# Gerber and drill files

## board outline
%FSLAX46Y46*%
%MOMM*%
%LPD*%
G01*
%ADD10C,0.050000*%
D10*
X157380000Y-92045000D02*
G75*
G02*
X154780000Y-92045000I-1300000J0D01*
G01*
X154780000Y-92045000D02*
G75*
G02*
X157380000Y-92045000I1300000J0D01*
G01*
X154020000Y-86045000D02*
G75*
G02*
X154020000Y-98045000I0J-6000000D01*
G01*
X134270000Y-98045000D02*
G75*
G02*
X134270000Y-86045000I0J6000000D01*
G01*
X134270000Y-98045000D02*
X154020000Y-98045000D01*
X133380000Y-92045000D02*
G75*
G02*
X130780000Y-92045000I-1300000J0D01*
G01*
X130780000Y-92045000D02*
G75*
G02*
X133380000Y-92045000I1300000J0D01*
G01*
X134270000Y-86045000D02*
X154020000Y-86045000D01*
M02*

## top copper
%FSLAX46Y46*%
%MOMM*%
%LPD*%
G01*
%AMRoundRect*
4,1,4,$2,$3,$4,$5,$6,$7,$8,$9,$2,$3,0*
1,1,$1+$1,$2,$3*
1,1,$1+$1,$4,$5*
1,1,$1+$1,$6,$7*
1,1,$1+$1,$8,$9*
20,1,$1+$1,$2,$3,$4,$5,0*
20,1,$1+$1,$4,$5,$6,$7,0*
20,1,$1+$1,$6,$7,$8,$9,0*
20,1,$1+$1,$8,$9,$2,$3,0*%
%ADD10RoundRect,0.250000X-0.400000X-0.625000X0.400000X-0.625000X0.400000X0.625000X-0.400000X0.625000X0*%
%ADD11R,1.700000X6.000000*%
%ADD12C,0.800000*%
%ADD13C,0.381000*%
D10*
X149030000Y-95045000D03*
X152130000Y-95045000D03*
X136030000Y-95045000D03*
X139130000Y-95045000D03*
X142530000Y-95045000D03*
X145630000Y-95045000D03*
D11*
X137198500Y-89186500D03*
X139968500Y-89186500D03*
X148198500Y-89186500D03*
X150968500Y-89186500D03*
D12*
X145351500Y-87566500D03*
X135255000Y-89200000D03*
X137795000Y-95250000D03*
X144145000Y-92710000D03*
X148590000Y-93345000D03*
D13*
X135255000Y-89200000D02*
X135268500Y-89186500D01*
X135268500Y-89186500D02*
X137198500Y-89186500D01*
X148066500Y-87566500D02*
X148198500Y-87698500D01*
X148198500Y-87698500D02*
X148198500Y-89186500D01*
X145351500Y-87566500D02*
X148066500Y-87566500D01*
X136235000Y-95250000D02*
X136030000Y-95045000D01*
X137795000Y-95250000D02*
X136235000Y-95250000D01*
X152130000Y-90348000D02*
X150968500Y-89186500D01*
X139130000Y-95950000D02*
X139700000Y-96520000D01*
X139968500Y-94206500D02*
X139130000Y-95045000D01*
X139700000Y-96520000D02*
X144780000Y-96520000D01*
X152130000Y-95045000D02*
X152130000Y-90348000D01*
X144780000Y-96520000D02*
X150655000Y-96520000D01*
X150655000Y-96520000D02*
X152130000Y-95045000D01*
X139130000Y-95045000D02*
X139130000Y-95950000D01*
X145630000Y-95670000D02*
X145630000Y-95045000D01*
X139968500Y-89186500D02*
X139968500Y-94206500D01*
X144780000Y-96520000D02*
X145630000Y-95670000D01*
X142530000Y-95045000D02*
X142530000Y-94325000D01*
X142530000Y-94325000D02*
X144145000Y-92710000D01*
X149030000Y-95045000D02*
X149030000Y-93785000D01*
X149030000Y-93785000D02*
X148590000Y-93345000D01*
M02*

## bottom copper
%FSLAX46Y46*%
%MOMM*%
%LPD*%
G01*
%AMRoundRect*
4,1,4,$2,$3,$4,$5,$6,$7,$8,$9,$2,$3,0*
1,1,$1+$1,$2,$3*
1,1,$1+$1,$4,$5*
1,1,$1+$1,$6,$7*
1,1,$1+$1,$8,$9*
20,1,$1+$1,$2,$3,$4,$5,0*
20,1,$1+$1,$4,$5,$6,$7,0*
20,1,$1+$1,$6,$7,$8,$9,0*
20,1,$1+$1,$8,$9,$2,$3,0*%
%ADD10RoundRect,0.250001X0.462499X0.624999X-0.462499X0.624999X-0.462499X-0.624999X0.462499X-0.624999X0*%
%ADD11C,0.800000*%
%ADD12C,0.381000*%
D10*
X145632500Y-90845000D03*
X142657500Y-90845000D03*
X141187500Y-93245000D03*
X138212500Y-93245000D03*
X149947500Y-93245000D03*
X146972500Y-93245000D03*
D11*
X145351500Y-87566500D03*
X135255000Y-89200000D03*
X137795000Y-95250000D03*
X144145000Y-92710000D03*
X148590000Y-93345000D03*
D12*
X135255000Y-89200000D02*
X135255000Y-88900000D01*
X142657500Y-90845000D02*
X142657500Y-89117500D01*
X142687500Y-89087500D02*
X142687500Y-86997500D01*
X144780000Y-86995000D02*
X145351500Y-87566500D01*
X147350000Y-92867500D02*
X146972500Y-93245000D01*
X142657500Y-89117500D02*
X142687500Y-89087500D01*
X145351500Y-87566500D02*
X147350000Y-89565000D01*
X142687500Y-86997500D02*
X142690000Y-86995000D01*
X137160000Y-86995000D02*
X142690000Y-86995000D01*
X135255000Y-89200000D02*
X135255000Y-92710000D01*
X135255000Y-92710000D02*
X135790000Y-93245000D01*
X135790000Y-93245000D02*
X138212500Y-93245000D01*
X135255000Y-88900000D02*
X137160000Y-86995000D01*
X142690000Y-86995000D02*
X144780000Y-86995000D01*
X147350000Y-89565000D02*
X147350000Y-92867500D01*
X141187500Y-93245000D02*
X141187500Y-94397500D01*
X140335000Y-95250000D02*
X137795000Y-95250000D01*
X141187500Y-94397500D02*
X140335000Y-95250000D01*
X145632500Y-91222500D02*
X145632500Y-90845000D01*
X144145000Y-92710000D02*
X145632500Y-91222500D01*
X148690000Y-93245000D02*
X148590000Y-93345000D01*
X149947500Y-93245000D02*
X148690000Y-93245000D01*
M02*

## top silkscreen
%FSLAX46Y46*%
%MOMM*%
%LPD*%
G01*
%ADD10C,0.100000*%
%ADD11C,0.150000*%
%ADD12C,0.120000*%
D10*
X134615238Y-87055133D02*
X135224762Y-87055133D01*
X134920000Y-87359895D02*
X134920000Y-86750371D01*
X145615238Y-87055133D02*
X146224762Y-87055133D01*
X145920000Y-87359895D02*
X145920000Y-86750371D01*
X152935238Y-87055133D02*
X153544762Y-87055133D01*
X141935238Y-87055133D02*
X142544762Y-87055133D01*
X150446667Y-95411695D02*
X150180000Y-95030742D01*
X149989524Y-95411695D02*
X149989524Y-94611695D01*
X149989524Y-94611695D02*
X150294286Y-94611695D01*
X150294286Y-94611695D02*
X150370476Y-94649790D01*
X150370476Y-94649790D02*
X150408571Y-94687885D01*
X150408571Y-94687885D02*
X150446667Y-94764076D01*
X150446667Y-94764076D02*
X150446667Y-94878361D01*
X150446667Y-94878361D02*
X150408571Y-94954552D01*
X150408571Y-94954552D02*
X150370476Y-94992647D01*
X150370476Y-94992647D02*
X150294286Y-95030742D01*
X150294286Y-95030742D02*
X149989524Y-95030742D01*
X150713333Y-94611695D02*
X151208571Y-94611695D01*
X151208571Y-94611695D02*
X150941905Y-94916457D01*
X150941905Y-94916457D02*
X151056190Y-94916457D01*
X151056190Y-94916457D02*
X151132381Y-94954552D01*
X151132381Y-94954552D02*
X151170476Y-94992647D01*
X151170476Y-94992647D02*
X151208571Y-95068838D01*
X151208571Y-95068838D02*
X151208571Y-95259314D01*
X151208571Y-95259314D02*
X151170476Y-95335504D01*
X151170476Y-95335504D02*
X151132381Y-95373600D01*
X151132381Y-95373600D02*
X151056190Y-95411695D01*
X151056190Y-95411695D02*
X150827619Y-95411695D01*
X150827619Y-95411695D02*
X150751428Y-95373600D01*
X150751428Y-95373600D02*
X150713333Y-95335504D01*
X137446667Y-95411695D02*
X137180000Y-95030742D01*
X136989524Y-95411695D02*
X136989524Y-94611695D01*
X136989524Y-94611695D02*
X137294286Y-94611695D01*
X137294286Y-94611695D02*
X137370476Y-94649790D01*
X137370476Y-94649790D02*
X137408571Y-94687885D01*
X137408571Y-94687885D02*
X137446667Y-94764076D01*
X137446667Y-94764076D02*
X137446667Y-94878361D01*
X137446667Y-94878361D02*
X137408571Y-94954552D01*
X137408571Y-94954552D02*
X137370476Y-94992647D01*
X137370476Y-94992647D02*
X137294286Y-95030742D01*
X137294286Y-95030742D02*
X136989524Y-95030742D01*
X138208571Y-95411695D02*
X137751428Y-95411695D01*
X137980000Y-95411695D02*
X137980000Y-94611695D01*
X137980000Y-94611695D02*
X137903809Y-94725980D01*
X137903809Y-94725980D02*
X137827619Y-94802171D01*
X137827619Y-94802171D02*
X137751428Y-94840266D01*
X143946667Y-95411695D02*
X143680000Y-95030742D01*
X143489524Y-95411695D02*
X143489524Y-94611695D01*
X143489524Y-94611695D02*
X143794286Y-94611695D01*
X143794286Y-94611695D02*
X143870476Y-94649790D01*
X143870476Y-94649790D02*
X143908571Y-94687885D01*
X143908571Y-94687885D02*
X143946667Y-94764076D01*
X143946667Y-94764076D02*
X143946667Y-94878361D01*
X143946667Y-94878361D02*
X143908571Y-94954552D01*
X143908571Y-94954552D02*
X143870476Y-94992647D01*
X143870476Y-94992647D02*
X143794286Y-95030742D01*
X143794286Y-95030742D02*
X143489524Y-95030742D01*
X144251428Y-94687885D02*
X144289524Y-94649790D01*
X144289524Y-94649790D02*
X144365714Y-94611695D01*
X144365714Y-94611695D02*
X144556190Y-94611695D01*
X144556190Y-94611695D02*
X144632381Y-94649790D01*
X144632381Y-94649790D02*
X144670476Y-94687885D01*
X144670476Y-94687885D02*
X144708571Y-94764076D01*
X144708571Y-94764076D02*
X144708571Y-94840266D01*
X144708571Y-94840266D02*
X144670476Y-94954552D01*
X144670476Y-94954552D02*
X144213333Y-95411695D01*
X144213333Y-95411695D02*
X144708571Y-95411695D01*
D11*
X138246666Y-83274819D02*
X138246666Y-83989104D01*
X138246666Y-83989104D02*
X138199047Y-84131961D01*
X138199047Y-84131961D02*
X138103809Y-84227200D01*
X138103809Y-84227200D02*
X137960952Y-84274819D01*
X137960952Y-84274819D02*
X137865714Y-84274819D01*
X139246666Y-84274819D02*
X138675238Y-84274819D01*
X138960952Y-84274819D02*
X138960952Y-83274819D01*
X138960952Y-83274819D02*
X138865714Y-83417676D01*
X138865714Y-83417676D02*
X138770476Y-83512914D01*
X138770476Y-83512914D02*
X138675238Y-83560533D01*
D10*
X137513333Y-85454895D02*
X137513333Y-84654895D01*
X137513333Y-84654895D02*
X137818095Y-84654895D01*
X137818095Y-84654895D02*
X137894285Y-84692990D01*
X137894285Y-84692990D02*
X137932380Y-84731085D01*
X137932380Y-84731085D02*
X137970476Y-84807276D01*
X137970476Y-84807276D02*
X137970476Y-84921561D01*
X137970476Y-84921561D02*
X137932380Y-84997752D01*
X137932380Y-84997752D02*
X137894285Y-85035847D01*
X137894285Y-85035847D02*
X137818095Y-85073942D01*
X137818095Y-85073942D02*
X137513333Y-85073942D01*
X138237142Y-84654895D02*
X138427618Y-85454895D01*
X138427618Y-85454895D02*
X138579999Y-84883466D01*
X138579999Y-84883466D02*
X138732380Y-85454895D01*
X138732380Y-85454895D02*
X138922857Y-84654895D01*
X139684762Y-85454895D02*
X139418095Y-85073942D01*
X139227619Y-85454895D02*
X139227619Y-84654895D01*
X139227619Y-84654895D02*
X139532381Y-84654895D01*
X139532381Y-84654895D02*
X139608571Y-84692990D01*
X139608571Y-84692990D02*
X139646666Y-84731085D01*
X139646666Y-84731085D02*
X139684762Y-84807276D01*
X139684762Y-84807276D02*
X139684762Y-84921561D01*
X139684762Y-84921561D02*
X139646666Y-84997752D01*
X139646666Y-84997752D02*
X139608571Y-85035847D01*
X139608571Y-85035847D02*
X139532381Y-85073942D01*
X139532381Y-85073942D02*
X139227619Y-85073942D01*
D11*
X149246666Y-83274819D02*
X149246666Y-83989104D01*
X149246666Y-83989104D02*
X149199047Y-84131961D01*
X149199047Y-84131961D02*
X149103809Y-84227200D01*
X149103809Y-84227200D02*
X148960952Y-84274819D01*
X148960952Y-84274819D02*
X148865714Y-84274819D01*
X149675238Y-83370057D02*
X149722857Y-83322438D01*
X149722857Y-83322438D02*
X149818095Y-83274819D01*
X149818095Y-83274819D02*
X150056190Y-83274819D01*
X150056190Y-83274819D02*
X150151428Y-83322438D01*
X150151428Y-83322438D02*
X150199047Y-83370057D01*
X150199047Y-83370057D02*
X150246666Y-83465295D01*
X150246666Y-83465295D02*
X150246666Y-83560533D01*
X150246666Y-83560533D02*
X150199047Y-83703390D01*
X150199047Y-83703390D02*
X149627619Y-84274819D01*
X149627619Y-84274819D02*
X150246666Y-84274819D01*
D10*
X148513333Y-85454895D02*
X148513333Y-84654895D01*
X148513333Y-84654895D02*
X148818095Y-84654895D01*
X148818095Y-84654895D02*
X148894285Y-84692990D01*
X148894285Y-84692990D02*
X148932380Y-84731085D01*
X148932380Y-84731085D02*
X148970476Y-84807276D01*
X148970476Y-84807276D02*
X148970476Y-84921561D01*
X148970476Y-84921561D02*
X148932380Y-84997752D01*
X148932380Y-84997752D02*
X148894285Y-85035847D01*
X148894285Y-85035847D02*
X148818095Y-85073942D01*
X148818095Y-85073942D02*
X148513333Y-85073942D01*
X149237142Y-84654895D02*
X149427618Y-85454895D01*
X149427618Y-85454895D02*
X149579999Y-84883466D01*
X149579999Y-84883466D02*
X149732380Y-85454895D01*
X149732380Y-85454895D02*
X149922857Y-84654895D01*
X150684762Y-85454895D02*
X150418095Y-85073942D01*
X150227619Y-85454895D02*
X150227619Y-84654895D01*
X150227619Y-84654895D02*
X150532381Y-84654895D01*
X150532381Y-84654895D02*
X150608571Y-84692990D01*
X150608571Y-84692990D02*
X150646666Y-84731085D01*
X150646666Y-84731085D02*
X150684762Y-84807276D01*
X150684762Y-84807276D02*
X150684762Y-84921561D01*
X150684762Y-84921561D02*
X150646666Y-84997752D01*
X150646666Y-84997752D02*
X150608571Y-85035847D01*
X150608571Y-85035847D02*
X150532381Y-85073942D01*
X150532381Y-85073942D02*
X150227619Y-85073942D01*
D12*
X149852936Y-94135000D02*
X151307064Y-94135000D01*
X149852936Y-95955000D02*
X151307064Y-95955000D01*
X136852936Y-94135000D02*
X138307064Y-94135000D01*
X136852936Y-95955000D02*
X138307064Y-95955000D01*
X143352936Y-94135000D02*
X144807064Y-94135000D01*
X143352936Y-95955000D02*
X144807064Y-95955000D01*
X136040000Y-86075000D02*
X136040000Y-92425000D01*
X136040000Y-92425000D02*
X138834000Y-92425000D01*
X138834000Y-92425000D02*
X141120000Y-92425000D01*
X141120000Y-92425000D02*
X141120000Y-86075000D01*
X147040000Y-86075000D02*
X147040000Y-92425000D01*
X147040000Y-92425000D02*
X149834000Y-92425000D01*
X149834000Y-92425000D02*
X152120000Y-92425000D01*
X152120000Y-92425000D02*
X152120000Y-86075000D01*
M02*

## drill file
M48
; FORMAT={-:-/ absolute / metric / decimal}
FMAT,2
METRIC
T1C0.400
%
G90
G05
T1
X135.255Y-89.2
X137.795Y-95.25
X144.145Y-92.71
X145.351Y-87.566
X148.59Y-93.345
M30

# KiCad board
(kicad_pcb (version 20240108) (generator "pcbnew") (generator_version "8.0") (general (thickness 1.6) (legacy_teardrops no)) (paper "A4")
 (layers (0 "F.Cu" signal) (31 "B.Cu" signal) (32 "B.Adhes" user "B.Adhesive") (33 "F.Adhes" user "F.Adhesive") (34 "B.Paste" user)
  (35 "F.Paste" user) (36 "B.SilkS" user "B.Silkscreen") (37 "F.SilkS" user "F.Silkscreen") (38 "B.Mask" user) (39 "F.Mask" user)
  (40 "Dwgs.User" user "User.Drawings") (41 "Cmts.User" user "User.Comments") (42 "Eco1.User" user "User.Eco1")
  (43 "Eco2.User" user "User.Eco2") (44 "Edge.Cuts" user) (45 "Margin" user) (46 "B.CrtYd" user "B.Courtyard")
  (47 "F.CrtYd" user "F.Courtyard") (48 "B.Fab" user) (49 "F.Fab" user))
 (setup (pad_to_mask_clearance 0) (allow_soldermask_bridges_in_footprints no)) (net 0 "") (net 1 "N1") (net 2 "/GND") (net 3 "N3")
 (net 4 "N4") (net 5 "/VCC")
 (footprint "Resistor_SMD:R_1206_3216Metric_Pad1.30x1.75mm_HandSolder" (layer "F.Cu") (at 150.58 95.045)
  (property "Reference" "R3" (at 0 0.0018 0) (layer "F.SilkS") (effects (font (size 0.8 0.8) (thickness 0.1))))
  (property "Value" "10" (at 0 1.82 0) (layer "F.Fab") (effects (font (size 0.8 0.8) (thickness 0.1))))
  (fp_line (start -0.727064 -0.91) (end 0.727064 -0.91) (stroke (width 0.12) (type solid)) (layer "F.SilkS"))
  (fp_line (start -0.727064 0.91) (end 0.727064 0.91) (stroke (width 0.12) (type solid)) (layer "F.SilkS"))
  (pad "1" smd roundrect (at -1.55 0) (size 1.3 1.75) (layers "F.Cu" "F.Paste" "F.Mask") (roundrect_rratio 0.192308) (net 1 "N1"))
  (pad "2" smd roundrect (at 1.55 0) (size 1.3 1.75) (layers "F.Cu" "F.Paste" "F.Mask") (roundrect_rratio 0.192308) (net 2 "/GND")))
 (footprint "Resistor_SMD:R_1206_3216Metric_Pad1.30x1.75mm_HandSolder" (layer "F.Cu") (at 137.58 95.045)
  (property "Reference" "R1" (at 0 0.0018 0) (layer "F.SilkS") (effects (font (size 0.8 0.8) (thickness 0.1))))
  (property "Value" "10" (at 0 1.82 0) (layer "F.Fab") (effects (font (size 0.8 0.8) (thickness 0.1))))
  (fp_line (start -0.727064 -0.91) (end 0.727064 -0.91) (stroke (width 0.12) (type solid)) (layer "F.SilkS"))
  (fp_line (start -0.727064 0.91) (end 0.727064 0.91) (stroke (width 0.12) (type solid)) (layer "F.SilkS"))
  (pad "1" smd roundrect (at -1.55 0) (size 1.3 1.75) (layers "F.Cu" "F.Paste" "F.Mask") (roundrect_rratio 0.192308) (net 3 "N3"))
  (pad "2" smd roundrect (at 1.55 0) (size 1.3 1.75) (layers "F.Cu" "F.Paste" "F.Mask") (roundrect_rratio 0.192308) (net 2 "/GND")))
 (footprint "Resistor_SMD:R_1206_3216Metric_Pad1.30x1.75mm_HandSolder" (layer "F.Cu") (at 144.08 95.045)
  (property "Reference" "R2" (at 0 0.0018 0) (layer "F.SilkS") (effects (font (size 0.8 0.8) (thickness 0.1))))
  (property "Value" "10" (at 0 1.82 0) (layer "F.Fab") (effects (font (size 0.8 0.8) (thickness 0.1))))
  (fp_line (start -0.727064 -0.91) (end 0.727064 -0.91) (stroke (width 0.12) (type solid)) (layer "F.SilkS"))
  (fp_line (start -0.727064 0.91) (end 0.727064 0.91) (stroke (width 0.12) (type solid)) (layer "F.SilkS"))
  (pad "1" smd roundrect (at -1.55 0) (size 1.3 1.75) (layers "F.Cu" "F.Paste" "F.Mask") (roundrect_rratio 0.192308) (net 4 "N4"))
  (pad "2" smd roundrect (at 1.55 0) (size 1.3 1.75) (layers "F.Cu" "F.Paste" "F.Mask") (roundrect_rratio 0.192308) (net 2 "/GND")))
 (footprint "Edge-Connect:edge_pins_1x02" (layer "F.Cu") (at 138.58 89.25 180)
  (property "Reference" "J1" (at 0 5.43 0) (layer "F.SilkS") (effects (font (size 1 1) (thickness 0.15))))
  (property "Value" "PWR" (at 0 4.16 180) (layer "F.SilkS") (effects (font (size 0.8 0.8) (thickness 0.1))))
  (fp_line (start 2.54 3.175) (end 2.54 -3.175) (stroke (width 0.12) (type solid)) (layer "F.SilkS"))
  (fp_line (start 2.54 -3.175) (end -0.254 -3.175) (stroke (width 0.12) (type solid)) (layer "F.SilkS"))
  (fp_line (start -0.254 -3.175) (end -2.54 -3.175) (stroke (width 0.12) (type solid)) (layer "F.SilkS"))
  (fp_line (start -2.54 -3.175) (end -2.54 3.175) (stroke (width 0.12) (type solid)) (layer "F.SilkS"))
  (pad "1" smd rect (at 1.3815 0.0635) (size 1.7 6) (layers "F.Cu" "F.Paste" "F.Mask") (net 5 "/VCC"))
  (pad "2" smd rect (at -1.3885 0.0635) (size 1.7 6) (layers "F.Cu" "F.Paste" "F.Mask") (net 2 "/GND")))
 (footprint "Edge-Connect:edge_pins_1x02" (layer "F.Cu") (at 149.58 89.25 180)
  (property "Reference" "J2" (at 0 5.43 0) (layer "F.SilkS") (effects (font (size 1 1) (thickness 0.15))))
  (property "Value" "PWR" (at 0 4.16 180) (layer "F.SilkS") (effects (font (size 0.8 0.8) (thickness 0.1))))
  (fp_line (start 2.54 3.175) (end 2.54 -3.175) (stroke (width 0.12) (type solid)) (layer "F.SilkS"))
  (fp_line (start 2.54 -3.175) (end -0.254 -3.175) (stroke (width 0.12) (type solid)) (layer "F.SilkS"))
  (fp_line (start -0.254 -3.175) (end -2.54 -3.175) (stroke (width 0.12) (type solid)) (layer "F.SilkS"))
  (fp_line (start -2.54 -3.175) (end -2.54 3.175) (stroke (width 0.12) (type solid)) (layer "F.SilkS"))
  (pad "1" smd rect (at 1.3815 0.0635) (size 1.7 6) (layers "F.Cu" "F.Paste" "F.Mask") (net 5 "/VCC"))
  (pad "2" smd rect (at -1.3885 0.0635) (size 1.7 6) (layers "F.Cu" "F.Paste" "F.Mask") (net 2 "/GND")))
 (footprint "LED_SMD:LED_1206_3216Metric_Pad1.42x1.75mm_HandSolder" (layer "B.Cu") (at 144.145 90.845 180)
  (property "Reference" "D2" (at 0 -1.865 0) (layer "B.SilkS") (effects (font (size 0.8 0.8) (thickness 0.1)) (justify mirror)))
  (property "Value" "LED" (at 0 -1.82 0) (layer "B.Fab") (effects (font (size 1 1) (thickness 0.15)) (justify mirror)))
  (pad "1" smd roundrect (at -1.4875 0 180) (size 1.425 1.75) (layers "B.Cu" "B.Paste" "B.Mask") (roundrect_rratio 0.175439) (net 4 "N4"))
  (pad "2" smd roundrect (at 1.4875 0 180) (size 1.425 1.75) (layers "B.Cu" "B.Paste" "B.Mask") (roundrect_rratio 0.175439) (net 5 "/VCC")))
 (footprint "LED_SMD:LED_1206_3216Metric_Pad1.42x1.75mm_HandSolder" (layer "B.Cu") (at 139.7 93.245 180)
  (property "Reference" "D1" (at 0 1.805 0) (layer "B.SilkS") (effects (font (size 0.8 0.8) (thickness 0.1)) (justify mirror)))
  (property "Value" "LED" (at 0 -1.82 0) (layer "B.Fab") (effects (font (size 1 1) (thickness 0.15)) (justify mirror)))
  (pad "1" smd roundrect (at -1.4875 0 180) (size 1.425 1.75) (layers "B.Cu" "B.Paste" "B.Mask") (roundrect_rratio 0.175439) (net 3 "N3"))
  (pad "2" smd roundrect (at 1.4875 0 180) (size 1.425 1.75) (layers "B.Cu" "B.Paste" "B.Mask") (roundrect_rratio 0.175439) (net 5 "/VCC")))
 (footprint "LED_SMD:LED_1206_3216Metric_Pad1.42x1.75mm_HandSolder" (layer "B.Cu") (at 148.46 93.245 180)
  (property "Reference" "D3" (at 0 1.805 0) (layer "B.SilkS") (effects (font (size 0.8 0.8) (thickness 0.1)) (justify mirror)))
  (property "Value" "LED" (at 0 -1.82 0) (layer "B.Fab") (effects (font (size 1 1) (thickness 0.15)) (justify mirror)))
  (pad "1" smd roundrect (at -1.4875 0 180) (size 1.425 1.75) (layers "B.Cu" "B.Paste" "B.Mask") (roundrect_rratio 0.175439) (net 1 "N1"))
  (pad "2" smd roundrect (at 1.4875 0 180) (size 1.425 1.75) (layers "B.Cu" "B.Paste" "B.Mask") (roundrect_rratio 0.175439) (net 5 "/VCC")))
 (gr_circle (center 156.08 92.045) (end 157.38 92.045) (stroke (width 0.05) (type default)) (fill none) (layer "Edge.Cuts"))
 (gr_arc (start 154.02 86.045) (mid 160.02 92.045) (end 154.02 98.045) (stroke (width 0.05) (type default)) (layer "Edge.Cuts"))
 (gr_arc (start 134.27 98.045) (mid 128.27 92.045) (end 134.27 86.045) (stroke (width 0.05) (type default)) (layer "Edge.Cuts"))
 (gr_line (start 134.27 98.045) (end 154.02 98.045) (stroke (width 0.05) (type default)) (layer "Edge.Cuts"))
 (gr_circle (center 132.08 92.045) (end 133.38 92.045) (stroke (width 0.05) (type default)) (fill none) (layer "Edge.Cuts"))
 (gr_line (start 134.27 86.045) (end 154.02 86.045) (stroke (width 0.05) (type default)) (layer "Edge.Cuts"))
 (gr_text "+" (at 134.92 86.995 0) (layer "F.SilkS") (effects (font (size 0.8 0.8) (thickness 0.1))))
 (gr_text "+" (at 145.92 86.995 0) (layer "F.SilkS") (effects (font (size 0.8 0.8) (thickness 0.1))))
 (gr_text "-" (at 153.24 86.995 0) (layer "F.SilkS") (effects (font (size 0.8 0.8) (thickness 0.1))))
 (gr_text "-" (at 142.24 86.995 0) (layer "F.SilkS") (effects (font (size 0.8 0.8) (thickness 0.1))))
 (segment (start 135.255 89.2) (end 135.2685 89.1865) (width 0.381) (layer "F.Cu") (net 5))
 (segment (start 135.2685 89.1865) (end 137.1985 89.1865) (width 0.381) (layer "F.Cu") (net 5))
 (segment (start 148.0665 87.5665) (end 148.1985 87.6985) (width 0.381) (layer "F.Cu") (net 5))
 (segment (start 148.1985 87.6985) (end 148.1985 89.1865) (width 0.381) (layer "F.Cu") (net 5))
 (segment (start 145.3515 87.5665) (end 148.0665 87.5665) (width 0.381) (layer "F.Cu") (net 5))
 (via (at 145.3515 87.5665) (size 0.8) (drill 0.4) (layers "F.Cu" "B.Cu") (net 5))
 (via (at 135.255 89.2) (size 0.8) (drill 0.4) (layers "F.Cu" "B.Cu") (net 5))
 (segment (start 135.255 89.2) (end 135.255 88.9) (width 0.381) (layer "B.Cu") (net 5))
 (segment (start 142.6575 90.845) (end 142.6575 89.1175) (width 0.381) (layer "B.Cu") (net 5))
 (segment (start 142.6875 89.0875) (end 142.6875 86.9975) (width 0.381) (layer "B.Cu") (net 5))
 (segment (start 144.78 86.995) (end 145.3515 87.5665) (width 0.381) (layer "B.Cu") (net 5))
 (segment (start 147.35 92.8675) (end 146.9725 93.245) (width 0.381) (layer "B.Cu") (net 5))
 (segment (start 142.6575 89.1175) (end 142.6875 89.0875) (width 0.381) (layer "B.Cu") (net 5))
 (segment (start 145.3515 87.5665) (end 147.35 89.565) (width 0.381) (layer "B.Cu") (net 5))
 (segment (start 142.6875 86.9975) (end 142.69 86.995) (width 0.381) (layer "B.Cu") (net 5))
 (segment (start 137.16 86.995) (end 142.69 86.995) (width 0.381) (layer "B.Cu") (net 5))
 (segment (start 135.255 89.2) (end 135.255 92.71) (width 0.381) (layer "B.Cu") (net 5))
 (segment (start 135.255 92.71) (end 135.79 93.245) (width 0.381) (layer "B.Cu") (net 5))
 (segment (start 135.79 93.245) (end 138.2125 93.245) (width 0.381) (layer "B.Cu") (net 5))
 (segment (start 135.255 88.9) (end 137.16 86.995) (width 0.381) (layer "B.Cu") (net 5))
 (segment (start 142.69 86.995) (end 144.78 86.995) (width 0.381) (layer "B.Cu") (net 5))
 (segment (start 147.35 89.565) (end 147.35 92.8675) (width 0.381) (layer "B.Cu") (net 5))
 (segment (start 136.235 95.25) (end 136.03 95.045) (width 0.381) (layer "F.Cu") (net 3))
 (segment (start 137.795 95.25) (end 136.235 95.25) (width 0.381) (layer "F.Cu") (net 3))
 (via (at 137.795 95.25) (size 0.8) (drill 0.4) (layers "F.Cu" "B.Cu") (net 3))
 (segment (start 141.1875 93.245) (end 141.1875 94.3975) (width 0.381) (layer "B.Cu") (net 3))
 (segment (start 140.335 95.25) (end 137.795 95.25) (width 0.381) (layer "B.Cu") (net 3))
 (segment (start 141.1875 94.3975) (end 140.335 95.25) (width 0.381) (layer "B.Cu") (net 3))
 (segment (start 152.13 90.348) (end 150.9685 89.1865) (width 0.381) (layer "F.Cu") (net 2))
 (segment (start 139.13 95.95) (end 139.7 96.52) (width 0.381) (layer "F.Cu") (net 2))
 (segment (start 139.9685 94.2065) (end 139.13 95.045) (width 0.381) (layer "F.Cu") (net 2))
 (segment (start 139.7 96.52) (end 144.78 96.52) (width 0.381) (layer "F.Cu") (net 2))
 (segment (start 152.13 95.045) (end 152.13 90.348) (width 0.381) (layer "F.Cu") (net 2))
 (segment (start 144.78 96.52) (end 150.655 96.52) (width 0.381) (layer "F.Cu") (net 2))
 (segment (start 150.655 96.52) (end 152.13 95.045) (width 0.381) (layer "F.Cu") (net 2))
 (segment (start 139.13 95.045) (end 139.13 95.95) (width 0.381) (layer "F.Cu") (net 2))
 (segment (start 145.63 95.67) (end 145.63 95.045) (width 0.381) (layer "F.Cu") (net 2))
 (segment (start 139.9685 89.1865) (end 139.9685 94.2065) (width 0.381) (layer "F.Cu") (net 2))
 (segment (start 144.78 96.52) (end 145.63 95.67) (width 0.381) (layer "F.Cu") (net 2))
 (segment (start 142.53 95.045) (end 142.53 94.325) (width 0.381) (layer "F.Cu") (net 4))
 (segment (start 142.53 94.325) (end 144.145 92.71) (width 0.381) (layer "F.Cu") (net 4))
 (via (at 144.145 92.71) (size 0.8) (drill 0.4) (layers "F.Cu" "B.Cu") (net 4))
 (segment (start 145.6325 91.2225) (end 145.6325 90.845) (width 0.381) (layer "B.Cu") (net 4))
 (segment (start 144.145 92.71) (end 145.6325 91.2225) (width 0.381) (layer "B.Cu") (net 4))
 (segment (start 149.03 95.045) (end 149.03 93.785) (width 0.381) (layer "F.Cu") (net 1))
 (segment (start 149.03 93.785) (end 148.59 93.345) (width 0.381) (layer "F.Cu") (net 1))
 (via (at 148.59 93.345) (size 0.8) (drill 0.4) (layers "F.Cu" "B.Cu") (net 1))
 (segment (start 148.69 93.245) (end 148.59 93.345) (width 0.381) (layer "B.Cu") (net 1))
 (segment (start 149.9475 93.245) (end 148.69 93.245) (width 0.381) (layer "B.Cu") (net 1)))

